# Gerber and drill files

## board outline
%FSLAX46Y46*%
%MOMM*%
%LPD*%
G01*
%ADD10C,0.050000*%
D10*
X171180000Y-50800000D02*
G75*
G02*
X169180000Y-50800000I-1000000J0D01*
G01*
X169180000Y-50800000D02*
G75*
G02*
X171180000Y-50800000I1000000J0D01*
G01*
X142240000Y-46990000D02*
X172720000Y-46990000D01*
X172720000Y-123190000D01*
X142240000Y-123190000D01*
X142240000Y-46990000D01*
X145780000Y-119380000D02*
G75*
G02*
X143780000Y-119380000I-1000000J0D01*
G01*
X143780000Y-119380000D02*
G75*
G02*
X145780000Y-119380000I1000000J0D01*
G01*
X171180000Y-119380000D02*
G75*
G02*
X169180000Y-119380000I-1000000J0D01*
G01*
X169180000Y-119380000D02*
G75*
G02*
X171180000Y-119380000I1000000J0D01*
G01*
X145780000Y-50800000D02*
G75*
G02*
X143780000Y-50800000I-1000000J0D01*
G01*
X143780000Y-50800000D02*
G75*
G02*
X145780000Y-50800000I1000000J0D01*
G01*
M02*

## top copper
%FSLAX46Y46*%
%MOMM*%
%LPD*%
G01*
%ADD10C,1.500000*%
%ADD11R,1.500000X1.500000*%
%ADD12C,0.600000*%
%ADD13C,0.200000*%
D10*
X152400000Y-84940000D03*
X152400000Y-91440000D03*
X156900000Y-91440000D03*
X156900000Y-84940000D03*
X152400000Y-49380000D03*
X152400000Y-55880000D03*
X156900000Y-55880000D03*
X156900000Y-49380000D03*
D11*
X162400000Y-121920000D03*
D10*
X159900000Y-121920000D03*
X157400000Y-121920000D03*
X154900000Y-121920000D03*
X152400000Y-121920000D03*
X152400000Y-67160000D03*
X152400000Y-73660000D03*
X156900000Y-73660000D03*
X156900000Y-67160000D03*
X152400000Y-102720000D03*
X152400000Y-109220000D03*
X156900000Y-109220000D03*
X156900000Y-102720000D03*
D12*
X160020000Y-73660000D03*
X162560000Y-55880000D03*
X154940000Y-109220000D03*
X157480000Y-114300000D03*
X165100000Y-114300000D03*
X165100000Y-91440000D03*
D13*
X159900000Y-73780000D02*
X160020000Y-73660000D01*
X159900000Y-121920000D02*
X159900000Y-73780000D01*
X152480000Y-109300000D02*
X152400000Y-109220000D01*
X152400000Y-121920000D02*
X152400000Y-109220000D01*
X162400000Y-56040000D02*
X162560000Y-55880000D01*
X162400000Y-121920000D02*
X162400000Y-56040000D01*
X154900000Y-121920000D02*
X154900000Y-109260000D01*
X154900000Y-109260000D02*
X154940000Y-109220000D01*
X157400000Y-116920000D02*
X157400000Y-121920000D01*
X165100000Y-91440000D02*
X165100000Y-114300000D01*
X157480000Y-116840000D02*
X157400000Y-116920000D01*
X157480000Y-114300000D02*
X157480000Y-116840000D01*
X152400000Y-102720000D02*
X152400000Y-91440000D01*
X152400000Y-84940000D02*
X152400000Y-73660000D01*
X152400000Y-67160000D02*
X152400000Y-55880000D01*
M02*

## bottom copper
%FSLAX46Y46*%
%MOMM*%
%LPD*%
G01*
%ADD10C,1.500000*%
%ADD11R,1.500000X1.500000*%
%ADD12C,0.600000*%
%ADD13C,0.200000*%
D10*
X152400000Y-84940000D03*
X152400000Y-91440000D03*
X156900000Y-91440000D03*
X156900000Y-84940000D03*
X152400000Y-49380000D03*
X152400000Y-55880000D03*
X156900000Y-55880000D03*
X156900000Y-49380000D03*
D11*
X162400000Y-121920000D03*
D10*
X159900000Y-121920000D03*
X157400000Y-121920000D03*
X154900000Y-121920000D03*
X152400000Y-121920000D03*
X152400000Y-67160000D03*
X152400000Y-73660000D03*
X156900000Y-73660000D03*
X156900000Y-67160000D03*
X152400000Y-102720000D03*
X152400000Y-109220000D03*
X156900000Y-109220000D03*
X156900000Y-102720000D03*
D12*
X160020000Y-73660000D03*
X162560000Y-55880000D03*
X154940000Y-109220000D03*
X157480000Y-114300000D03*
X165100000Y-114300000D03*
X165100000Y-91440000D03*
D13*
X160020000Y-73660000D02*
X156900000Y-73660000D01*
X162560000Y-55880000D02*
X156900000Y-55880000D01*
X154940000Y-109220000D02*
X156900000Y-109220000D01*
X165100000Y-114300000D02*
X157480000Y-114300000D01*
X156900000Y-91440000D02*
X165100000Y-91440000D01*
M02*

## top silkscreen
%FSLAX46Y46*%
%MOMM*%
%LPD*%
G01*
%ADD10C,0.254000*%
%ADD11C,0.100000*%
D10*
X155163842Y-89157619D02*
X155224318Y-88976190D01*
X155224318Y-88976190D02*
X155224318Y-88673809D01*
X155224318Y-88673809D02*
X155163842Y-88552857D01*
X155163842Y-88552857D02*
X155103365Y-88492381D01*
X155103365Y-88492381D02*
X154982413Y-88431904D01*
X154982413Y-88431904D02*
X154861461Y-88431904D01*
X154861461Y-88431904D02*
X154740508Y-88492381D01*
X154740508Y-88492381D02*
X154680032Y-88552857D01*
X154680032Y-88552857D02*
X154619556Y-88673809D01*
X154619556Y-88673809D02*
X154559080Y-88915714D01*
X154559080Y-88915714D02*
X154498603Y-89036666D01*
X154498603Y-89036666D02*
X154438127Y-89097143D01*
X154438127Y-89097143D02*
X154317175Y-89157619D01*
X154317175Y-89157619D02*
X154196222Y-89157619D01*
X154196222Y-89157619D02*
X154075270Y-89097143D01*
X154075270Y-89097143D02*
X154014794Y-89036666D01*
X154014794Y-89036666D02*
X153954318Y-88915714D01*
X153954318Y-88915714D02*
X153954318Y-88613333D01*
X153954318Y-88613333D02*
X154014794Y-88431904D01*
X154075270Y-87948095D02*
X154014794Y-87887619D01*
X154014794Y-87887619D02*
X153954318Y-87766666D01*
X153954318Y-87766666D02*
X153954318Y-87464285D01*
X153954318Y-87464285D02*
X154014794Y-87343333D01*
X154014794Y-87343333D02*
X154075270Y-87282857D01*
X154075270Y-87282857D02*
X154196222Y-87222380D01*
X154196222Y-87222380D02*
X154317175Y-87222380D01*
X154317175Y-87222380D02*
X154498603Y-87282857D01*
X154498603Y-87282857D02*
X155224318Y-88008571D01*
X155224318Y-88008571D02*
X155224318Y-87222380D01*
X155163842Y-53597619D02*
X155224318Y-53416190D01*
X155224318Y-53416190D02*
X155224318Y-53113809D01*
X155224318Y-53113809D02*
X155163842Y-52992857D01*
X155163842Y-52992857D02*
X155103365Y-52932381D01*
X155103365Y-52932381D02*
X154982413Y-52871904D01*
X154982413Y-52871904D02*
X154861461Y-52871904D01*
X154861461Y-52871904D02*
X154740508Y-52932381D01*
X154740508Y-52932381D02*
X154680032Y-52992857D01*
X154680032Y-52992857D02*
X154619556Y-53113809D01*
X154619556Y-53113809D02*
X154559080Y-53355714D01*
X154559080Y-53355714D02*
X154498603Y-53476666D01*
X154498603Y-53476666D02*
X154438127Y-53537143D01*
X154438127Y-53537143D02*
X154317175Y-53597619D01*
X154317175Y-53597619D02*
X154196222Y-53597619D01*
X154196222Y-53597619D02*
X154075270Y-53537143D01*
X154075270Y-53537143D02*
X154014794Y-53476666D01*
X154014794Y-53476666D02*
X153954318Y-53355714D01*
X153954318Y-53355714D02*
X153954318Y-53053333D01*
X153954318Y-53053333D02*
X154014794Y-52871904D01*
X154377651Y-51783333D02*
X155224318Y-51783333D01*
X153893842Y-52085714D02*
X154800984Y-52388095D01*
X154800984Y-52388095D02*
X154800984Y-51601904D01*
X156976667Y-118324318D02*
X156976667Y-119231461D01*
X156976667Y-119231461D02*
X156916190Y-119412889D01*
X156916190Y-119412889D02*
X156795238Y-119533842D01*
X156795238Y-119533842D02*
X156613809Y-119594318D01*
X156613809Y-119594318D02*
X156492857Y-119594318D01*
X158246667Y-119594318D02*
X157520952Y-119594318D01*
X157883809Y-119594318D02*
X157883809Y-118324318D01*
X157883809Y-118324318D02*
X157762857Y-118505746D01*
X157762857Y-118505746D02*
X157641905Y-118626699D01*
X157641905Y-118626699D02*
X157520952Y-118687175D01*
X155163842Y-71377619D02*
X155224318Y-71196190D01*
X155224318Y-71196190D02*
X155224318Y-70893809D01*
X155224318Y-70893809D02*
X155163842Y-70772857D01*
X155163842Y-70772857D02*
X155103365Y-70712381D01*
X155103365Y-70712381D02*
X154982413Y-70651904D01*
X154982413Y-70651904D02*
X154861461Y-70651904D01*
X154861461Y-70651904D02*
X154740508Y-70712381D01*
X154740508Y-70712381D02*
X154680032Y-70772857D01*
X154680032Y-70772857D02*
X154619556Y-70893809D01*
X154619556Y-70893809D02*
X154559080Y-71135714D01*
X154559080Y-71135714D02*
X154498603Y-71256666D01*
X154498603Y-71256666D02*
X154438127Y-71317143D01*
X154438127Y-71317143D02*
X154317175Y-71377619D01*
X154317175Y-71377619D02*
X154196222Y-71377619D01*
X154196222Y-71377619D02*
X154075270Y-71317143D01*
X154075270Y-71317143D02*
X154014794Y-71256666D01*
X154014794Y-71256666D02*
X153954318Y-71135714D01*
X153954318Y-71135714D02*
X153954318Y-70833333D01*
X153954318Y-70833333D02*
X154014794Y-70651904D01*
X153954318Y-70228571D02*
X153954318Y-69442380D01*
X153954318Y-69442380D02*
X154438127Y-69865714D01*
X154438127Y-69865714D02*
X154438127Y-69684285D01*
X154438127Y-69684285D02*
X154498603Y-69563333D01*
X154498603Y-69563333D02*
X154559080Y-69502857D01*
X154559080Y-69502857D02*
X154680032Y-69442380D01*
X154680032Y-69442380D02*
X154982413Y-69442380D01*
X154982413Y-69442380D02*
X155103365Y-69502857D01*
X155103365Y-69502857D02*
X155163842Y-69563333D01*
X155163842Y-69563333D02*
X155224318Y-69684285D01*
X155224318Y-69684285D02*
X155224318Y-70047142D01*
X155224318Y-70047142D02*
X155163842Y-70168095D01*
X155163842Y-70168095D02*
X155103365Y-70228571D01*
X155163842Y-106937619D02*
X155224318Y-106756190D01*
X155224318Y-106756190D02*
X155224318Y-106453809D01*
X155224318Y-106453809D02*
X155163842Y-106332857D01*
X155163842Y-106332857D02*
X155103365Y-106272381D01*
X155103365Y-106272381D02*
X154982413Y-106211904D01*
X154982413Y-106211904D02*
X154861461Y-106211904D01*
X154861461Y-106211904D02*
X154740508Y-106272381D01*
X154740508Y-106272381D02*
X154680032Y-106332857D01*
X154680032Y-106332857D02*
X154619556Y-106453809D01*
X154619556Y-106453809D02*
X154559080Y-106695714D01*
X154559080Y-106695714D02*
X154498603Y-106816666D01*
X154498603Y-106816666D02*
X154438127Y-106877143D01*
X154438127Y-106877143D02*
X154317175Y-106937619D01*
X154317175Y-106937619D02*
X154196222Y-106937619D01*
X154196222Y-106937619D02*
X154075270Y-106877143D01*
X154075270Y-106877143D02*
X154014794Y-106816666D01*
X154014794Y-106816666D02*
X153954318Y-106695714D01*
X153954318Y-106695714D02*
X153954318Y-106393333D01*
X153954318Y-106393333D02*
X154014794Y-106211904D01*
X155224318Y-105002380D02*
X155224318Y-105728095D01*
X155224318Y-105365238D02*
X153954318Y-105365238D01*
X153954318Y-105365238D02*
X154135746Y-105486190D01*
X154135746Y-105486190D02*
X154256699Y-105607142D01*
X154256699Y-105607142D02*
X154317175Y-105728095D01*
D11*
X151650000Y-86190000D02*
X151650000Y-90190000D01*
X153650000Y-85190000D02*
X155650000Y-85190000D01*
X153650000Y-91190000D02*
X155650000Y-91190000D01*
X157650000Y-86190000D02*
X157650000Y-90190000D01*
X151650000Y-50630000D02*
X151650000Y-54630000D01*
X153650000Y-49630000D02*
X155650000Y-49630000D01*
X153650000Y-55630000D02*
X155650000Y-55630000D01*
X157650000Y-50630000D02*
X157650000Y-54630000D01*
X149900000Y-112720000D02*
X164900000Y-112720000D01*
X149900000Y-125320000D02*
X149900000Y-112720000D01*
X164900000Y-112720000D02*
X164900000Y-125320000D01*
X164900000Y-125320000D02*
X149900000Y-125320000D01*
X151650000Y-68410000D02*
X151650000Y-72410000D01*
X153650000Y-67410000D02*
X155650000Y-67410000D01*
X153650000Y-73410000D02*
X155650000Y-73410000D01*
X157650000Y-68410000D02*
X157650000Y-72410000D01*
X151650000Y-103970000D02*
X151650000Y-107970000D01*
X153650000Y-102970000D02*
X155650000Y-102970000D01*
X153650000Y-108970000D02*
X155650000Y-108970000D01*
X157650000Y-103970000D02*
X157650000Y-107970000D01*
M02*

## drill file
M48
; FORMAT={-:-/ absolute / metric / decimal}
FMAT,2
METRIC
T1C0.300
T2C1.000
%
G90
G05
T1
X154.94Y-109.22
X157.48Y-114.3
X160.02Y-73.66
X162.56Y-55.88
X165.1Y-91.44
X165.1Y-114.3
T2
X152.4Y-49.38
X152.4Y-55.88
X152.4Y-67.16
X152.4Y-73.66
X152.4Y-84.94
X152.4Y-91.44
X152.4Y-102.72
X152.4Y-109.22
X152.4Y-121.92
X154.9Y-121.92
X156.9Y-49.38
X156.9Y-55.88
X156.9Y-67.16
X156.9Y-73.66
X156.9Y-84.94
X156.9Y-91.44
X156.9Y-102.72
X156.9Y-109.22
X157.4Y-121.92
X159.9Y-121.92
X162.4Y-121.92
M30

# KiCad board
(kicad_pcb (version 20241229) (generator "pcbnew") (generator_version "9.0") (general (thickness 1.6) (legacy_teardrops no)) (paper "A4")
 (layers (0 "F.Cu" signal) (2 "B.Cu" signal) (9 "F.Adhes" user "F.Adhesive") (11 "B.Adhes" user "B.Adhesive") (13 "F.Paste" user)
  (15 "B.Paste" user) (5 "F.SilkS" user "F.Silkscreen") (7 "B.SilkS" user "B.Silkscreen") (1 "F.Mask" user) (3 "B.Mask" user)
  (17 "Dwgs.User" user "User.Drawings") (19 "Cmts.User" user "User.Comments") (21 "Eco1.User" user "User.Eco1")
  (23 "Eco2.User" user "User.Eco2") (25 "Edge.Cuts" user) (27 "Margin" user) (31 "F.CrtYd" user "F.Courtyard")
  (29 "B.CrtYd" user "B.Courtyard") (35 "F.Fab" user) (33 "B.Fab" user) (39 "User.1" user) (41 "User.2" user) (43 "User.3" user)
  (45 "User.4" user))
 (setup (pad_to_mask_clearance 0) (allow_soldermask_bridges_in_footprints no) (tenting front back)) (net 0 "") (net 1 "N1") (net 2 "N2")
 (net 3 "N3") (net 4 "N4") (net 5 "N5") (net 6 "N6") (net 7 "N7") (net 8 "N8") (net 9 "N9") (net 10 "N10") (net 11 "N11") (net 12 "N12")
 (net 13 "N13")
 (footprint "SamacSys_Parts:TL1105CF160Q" (layer "F.Cu") (at 154.65 88.19 -90)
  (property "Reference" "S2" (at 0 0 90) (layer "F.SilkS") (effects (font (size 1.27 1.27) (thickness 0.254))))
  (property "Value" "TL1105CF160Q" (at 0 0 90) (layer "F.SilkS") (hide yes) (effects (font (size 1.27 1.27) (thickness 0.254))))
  (fp_line (start -2 3) (end 2 3) (stroke (width 0.1) (type solid)) (layer "F.SilkS"))
  (fp_line (start -3 1) (end -3 -1) (stroke (width 0.1) (type solid)) (layer "F.SilkS"))
  (fp_line (start 3 1) (end 3 -1) (stroke (width 0.1) (type solid)) (layer "F.SilkS"))
  (fp_line (start -2 -3) (end 2 -3) (stroke (width 0.1) (type solid)) (layer "F.SilkS"))
  (pad "1" thru_hole circle (at -3.25 2.25 270) (size 1.5 1.5) (drill 1) (layers "*.Cu" "*.Mask") (remove_unused_layers no) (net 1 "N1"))
  (pad "2" thru_hole circle (at 3.25 2.25 270) (size 1.5 1.5) (drill 1) (layers "*.Cu" "*.Mask") (remove_unused_layers no) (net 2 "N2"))
  (pad "3" thru_hole circle (at 3.25 -2.25 270) (size 1.5 1.5) (drill 1) (layers "*.Cu" "*.Mask") (remove_unused_layers no) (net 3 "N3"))
  (pad "4" thru_hole circle (at -3.25 -2.25 270) (size 1.5 1.5) (drill 1) (layers "*.Cu" "*.Mask") (remove_unused_layers no) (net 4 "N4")))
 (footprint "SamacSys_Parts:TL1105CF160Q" (layer "F.Cu") (at 154.65 52.63 -90)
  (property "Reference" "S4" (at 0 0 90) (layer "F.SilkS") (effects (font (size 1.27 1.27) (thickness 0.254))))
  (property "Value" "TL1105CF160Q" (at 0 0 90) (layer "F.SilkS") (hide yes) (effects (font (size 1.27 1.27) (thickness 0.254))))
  (fp_line (start -2 3) (end 2 3) (stroke (width 0.1) (type solid)) (layer "F.SilkS"))
  (fp_line (start -3 1) (end -3 -1) (stroke (width 0.1) (type solid)) (layer "F.SilkS"))
  (fp_line (start 3 1) (end 3 -1) (stroke (width 0.1) (type solid)) (layer "F.SilkS"))
  (fp_line (start -2 -3) (end 2 -3) (stroke (width 0.1) (type solid)) (layer "F.SilkS"))
  (pad "1" thru_hole circle (at -3.25 2.25 270) (size 1.5 1.5) (drill 1) (layers "*.Cu" "*.Mask") (remove_unused_layers no) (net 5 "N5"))
  (pad "2" thru_hole circle (at 3.25 2.25 270) (size 1.5 1.5) (drill 1) (layers "*.Cu" "*.Mask") (remove_unused_layers no) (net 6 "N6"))
  (pad "3" thru_hole circle (at 3.25 -2.25 270) (size 1.5 1.5) (drill 1) (layers "*.Cu" "*.Mask") (remove_unused_layers no) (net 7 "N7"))
  (pad "4" thru_hole circle (at -3.25 -2.25 270) (size 1.5 1.5) (drill 1) (layers "*.Cu" "*.Mask") (remove_unused_layers no) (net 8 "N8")))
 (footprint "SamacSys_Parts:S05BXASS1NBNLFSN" (layer "F.Cu") (at 162.4 121.92 180)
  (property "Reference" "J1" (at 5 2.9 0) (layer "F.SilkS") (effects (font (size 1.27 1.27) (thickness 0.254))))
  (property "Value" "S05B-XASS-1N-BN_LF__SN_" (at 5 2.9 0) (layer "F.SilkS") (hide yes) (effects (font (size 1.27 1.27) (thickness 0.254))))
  (fp_line (start 12.5 9.2) (end -2.5 9.2) (stroke (width 0.1) (type solid)) (layer "F.SilkS"))
  (fp_line (start 12.5 -3.4) (end 12.5 9.2) (stroke (width 0.1) (type solid)) (layer "F.SilkS"))
  (fp_line (start -2.5 9.2) (end -2.5 -3.4) (stroke (width 0.1) (type solid)) (layer "F.SilkS"))
  (fp_line (start -2.5 -3.4) (end 12.5 -3.4) (stroke (width 0.1) (type solid)) (layer "F.SilkS"))
  (pad "1" thru_hole rect (at 0 0 180) (size 1.5 1.5) (drill 1) (layers "*.Cu" "*.Mask") (remove_unused_layers no) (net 7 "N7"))
  (pad "2" thru_hole circle (at 2.5 0 180) (size 1.5 1.5) (drill 1) (layers "*.Cu" "*.Mask") (remove_unused_layers no) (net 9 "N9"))
  (pad "3" thru_hole circle (at 5 0 180) (size 1.5 1.5) (drill 1) (layers "*.Cu" "*.Mask") (remove_unused_layers no) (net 3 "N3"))
  (pad "4" thru_hole circle (at 7.5 0 180) (size 1.5 1.5) (drill 1) (layers "*.Cu" "*.Mask") (remove_unused_layers no) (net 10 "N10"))
  (pad "5" thru_hole circle (at 10 0 180) (size 1.5 1.5) (drill 1) (layers "*.Cu" "*.Mask") (remove_unused_layers no) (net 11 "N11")))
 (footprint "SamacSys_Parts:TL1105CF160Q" (layer "F.Cu") (at 154.65 70.41 -90)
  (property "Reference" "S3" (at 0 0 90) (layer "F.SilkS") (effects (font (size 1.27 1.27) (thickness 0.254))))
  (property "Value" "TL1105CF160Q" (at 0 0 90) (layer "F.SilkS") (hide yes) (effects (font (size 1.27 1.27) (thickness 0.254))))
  (fp_line (start -2 3) (end 2 3) (stroke (width 0.1) (type solid)) (layer "F.SilkS"))
  (fp_line (start -3 1) (end -3 -1) (stroke (width 0.1) (type solid)) (layer "F.SilkS"))
  (fp_line (start 3 1) (end 3 -1) (stroke (width 0.1) (type solid)) (layer "F.SilkS"))
  (fp_line (start -2 -3) (end 2 -3) (stroke (width 0.1) (type solid)) (layer "F.SilkS"))
  (pad "1" thru_hole circle (at -3.25 2.25 270) (size 1.5 1.5) (drill 1) (layers "*.Cu" "*.Mask") (remove_unused_layers no) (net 6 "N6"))
  (pad "2" thru_hole circle (at 3.25 2.25 270) (size 1.5 1.5) (drill 1) (layers "*.Cu" "*.Mask") (remove_unused_layers no) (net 1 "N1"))
  (pad "3" thru_hole circle (at 3.25 -2.25 270) (size 1.5 1.5) (drill 1) (layers "*.Cu" "*.Mask") (remove_unused_layers no) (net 9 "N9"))
  (pad "4" thru_hole circle (at -3.25 -2.25 270) (size 1.5 1.5) (drill 1) (layers "*.Cu" "*.Mask") (remove_unused_layers no) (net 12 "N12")))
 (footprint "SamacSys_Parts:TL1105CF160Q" (layer "F.Cu") (at 154.65 105.97 -90)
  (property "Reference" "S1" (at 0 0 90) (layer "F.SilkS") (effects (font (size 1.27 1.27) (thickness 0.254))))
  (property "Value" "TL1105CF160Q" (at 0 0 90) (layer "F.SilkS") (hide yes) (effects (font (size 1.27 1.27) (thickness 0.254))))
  (fp_line (start -2 3) (end 2 3) (stroke (width 0.1) (type solid)) (layer "F.SilkS"))
  (fp_line (start -3 1) (end -3 -1) (stroke (width 0.1) (type solid)) (layer "F.SilkS"))
  (fp_line (start 3 1) (end 3 -1) (stroke (width 0.1) (type solid)) (layer "F.SilkS"))
  (fp_line (start -2 -3) (end 2 -3) (stroke (width 0.1) (type solid)) (layer "F.SilkS"))
  (pad "1" thru_hole circle (at -3.25 2.25 270) (size 1.5 1.5) (drill 1) (layers "*.Cu" "*.Mask") (remove_unused_layers no) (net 2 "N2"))
  (pad "2" thru_hole circle (at 3.25 2.25 270) (size 1.5 1.5) (drill 1) (layers "*.Cu" "*.Mask") (remove_unused_layers no) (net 11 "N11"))
  (pad "3" thru_hole circle (at 3.25 -2.25 270) (size 1.5 1.5) (drill 1) (layers "*.Cu" "*.Mask") (remove_unused_layers no) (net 10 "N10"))
  (pad "4" thru_hole circle (at -3.25 -2.25 270) (size 1.5 1.5) (drill 1) (layers "*.Cu" "*.Mask") (remove_unused_layers no) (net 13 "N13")))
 (gr_circle (center 170.18 50.8) (end 171.18 50.8) (stroke (width 0.05) (type default)) (fill no) (layer "Edge.Cuts"))
 (gr_rect (start 142.24 46.99) (end 172.72 123.19) (stroke (width 0.05) (type default)) (fill no) (layer "Edge.Cuts"))
 (gr_circle (center 144.78 119.38) (end 145.78 119.38) (stroke (width 0.05) (type default)) (fill no) (layer "Edge.Cuts"))
 (gr_circle (center 170.18 119.38) (end 171.18 119.38) (stroke (width 0.05) (type default)) (fill no) (layer "Edge.Cuts"))
 (gr_circle (center 144.78 50.8) (end 145.78 50.8) (stroke (width 0.05) (type default)) (fill no) (layer "Edge.Cuts"))
 (segment (start 159.9 73.78) (end 160.02 73.66) (width 0.2) (layer "F.Cu") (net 9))
 (segment (start 159.9 121.92) (end 159.9 73.78) (width 0.2) (layer "F.Cu") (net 9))
 (via (at 160.02 73.66) (size 0.6) (drill 0.3) (layers "F.Cu" "B.Cu") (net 9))
 (segment (start 160.02 73.66) (end 156.9 73.66) (width 0.2) (layer "B.Cu") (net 9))
 (segment (start 152.48 109.3) (end 152.4 109.22) (width 0.2) (layer "F.Cu") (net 11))
 (segment (start 152.4 121.92) (end 152.4 109.22) (width 0.2) (layer "F.Cu") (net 11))
 (segment (start 162.4 56.04) (end 162.56 55.88) (width 0.2) (layer "F.Cu") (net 7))
 (segment (start 162.4 121.92) (end 162.4 56.04) (width 0.2) (layer "F.Cu") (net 7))
 (via (at 162.56 55.88) (size 0.6) (drill 0.3) (layers "F.Cu" "B.Cu") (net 7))
 (segment (start 162.56 55.88) (end 156.9 55.88) (width 0.2) (layer "B.Cu") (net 7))
 (segment (start 154.9 121.92) (end 154.9 109.26) (width 0.2) (layer "F.Cu") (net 10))
 (segment (start 154.9 109.26) (end 154.94 109.22) (width 0.2) (layer "F.Cu") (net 10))
 (via (at 154.94 109.22) (size 0.6) (drill 0.3) (layers "F.Cu" "B.Cu") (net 10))
 (segment (start 154.94 109.22) (end 156.9 109.22) (width 0.2) (layer "B.Cu") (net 10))
 (segment (start 157.4 116.92) (end 157.4 121.92) (width 0.2) (layer "F.Cu") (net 3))
 (segment (start 165.1 91.44) (end 165.1 114.3) (width 0.2) (layer "F.Cu") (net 3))
 (segment (start 157.48 116.84) (end 157.4 116.92) (width 0.2) (layer "F.Cu") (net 3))
 (segment (start 157.48 114.3) (end 157.48 116.84) (width 0.2) (layer "F.Cu") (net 3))
 (via (at 157.48 114.3) (size 0.6) (drill 0.3) (layers "F.Cu" "B.Cu") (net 3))
 (via (at 165.1 114.3) (size 0.6) (drill 0.3) (layers "F.Cu" "B.Cu") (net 3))
 (via (at 165.1 91.44) (size 0.6) (drill 0.3) (layers "F.Cu" "B.Cu") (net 3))
 (segment (start 165.1 114.3) (end 157.48 114.3) (width 0.2) (layer "B.Cu") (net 3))
 (segment (start 156.9 91.44) (end 165.1 91.44) (width 0.2) (layer "B.Cu") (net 3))
 (segment (start 152.4 102.72) (end 152.4 91.44) (width 0.2) (layer "F.Cu") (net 2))
 (segment (start 152.4 84.94) (end 152.4 73.66) (width 0.2) (layer "F.Cu") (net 1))
 (segment (start 152.4 67.16) (end 152.4 55.88) (width 0.2) (layer "F.Cu") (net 6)))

